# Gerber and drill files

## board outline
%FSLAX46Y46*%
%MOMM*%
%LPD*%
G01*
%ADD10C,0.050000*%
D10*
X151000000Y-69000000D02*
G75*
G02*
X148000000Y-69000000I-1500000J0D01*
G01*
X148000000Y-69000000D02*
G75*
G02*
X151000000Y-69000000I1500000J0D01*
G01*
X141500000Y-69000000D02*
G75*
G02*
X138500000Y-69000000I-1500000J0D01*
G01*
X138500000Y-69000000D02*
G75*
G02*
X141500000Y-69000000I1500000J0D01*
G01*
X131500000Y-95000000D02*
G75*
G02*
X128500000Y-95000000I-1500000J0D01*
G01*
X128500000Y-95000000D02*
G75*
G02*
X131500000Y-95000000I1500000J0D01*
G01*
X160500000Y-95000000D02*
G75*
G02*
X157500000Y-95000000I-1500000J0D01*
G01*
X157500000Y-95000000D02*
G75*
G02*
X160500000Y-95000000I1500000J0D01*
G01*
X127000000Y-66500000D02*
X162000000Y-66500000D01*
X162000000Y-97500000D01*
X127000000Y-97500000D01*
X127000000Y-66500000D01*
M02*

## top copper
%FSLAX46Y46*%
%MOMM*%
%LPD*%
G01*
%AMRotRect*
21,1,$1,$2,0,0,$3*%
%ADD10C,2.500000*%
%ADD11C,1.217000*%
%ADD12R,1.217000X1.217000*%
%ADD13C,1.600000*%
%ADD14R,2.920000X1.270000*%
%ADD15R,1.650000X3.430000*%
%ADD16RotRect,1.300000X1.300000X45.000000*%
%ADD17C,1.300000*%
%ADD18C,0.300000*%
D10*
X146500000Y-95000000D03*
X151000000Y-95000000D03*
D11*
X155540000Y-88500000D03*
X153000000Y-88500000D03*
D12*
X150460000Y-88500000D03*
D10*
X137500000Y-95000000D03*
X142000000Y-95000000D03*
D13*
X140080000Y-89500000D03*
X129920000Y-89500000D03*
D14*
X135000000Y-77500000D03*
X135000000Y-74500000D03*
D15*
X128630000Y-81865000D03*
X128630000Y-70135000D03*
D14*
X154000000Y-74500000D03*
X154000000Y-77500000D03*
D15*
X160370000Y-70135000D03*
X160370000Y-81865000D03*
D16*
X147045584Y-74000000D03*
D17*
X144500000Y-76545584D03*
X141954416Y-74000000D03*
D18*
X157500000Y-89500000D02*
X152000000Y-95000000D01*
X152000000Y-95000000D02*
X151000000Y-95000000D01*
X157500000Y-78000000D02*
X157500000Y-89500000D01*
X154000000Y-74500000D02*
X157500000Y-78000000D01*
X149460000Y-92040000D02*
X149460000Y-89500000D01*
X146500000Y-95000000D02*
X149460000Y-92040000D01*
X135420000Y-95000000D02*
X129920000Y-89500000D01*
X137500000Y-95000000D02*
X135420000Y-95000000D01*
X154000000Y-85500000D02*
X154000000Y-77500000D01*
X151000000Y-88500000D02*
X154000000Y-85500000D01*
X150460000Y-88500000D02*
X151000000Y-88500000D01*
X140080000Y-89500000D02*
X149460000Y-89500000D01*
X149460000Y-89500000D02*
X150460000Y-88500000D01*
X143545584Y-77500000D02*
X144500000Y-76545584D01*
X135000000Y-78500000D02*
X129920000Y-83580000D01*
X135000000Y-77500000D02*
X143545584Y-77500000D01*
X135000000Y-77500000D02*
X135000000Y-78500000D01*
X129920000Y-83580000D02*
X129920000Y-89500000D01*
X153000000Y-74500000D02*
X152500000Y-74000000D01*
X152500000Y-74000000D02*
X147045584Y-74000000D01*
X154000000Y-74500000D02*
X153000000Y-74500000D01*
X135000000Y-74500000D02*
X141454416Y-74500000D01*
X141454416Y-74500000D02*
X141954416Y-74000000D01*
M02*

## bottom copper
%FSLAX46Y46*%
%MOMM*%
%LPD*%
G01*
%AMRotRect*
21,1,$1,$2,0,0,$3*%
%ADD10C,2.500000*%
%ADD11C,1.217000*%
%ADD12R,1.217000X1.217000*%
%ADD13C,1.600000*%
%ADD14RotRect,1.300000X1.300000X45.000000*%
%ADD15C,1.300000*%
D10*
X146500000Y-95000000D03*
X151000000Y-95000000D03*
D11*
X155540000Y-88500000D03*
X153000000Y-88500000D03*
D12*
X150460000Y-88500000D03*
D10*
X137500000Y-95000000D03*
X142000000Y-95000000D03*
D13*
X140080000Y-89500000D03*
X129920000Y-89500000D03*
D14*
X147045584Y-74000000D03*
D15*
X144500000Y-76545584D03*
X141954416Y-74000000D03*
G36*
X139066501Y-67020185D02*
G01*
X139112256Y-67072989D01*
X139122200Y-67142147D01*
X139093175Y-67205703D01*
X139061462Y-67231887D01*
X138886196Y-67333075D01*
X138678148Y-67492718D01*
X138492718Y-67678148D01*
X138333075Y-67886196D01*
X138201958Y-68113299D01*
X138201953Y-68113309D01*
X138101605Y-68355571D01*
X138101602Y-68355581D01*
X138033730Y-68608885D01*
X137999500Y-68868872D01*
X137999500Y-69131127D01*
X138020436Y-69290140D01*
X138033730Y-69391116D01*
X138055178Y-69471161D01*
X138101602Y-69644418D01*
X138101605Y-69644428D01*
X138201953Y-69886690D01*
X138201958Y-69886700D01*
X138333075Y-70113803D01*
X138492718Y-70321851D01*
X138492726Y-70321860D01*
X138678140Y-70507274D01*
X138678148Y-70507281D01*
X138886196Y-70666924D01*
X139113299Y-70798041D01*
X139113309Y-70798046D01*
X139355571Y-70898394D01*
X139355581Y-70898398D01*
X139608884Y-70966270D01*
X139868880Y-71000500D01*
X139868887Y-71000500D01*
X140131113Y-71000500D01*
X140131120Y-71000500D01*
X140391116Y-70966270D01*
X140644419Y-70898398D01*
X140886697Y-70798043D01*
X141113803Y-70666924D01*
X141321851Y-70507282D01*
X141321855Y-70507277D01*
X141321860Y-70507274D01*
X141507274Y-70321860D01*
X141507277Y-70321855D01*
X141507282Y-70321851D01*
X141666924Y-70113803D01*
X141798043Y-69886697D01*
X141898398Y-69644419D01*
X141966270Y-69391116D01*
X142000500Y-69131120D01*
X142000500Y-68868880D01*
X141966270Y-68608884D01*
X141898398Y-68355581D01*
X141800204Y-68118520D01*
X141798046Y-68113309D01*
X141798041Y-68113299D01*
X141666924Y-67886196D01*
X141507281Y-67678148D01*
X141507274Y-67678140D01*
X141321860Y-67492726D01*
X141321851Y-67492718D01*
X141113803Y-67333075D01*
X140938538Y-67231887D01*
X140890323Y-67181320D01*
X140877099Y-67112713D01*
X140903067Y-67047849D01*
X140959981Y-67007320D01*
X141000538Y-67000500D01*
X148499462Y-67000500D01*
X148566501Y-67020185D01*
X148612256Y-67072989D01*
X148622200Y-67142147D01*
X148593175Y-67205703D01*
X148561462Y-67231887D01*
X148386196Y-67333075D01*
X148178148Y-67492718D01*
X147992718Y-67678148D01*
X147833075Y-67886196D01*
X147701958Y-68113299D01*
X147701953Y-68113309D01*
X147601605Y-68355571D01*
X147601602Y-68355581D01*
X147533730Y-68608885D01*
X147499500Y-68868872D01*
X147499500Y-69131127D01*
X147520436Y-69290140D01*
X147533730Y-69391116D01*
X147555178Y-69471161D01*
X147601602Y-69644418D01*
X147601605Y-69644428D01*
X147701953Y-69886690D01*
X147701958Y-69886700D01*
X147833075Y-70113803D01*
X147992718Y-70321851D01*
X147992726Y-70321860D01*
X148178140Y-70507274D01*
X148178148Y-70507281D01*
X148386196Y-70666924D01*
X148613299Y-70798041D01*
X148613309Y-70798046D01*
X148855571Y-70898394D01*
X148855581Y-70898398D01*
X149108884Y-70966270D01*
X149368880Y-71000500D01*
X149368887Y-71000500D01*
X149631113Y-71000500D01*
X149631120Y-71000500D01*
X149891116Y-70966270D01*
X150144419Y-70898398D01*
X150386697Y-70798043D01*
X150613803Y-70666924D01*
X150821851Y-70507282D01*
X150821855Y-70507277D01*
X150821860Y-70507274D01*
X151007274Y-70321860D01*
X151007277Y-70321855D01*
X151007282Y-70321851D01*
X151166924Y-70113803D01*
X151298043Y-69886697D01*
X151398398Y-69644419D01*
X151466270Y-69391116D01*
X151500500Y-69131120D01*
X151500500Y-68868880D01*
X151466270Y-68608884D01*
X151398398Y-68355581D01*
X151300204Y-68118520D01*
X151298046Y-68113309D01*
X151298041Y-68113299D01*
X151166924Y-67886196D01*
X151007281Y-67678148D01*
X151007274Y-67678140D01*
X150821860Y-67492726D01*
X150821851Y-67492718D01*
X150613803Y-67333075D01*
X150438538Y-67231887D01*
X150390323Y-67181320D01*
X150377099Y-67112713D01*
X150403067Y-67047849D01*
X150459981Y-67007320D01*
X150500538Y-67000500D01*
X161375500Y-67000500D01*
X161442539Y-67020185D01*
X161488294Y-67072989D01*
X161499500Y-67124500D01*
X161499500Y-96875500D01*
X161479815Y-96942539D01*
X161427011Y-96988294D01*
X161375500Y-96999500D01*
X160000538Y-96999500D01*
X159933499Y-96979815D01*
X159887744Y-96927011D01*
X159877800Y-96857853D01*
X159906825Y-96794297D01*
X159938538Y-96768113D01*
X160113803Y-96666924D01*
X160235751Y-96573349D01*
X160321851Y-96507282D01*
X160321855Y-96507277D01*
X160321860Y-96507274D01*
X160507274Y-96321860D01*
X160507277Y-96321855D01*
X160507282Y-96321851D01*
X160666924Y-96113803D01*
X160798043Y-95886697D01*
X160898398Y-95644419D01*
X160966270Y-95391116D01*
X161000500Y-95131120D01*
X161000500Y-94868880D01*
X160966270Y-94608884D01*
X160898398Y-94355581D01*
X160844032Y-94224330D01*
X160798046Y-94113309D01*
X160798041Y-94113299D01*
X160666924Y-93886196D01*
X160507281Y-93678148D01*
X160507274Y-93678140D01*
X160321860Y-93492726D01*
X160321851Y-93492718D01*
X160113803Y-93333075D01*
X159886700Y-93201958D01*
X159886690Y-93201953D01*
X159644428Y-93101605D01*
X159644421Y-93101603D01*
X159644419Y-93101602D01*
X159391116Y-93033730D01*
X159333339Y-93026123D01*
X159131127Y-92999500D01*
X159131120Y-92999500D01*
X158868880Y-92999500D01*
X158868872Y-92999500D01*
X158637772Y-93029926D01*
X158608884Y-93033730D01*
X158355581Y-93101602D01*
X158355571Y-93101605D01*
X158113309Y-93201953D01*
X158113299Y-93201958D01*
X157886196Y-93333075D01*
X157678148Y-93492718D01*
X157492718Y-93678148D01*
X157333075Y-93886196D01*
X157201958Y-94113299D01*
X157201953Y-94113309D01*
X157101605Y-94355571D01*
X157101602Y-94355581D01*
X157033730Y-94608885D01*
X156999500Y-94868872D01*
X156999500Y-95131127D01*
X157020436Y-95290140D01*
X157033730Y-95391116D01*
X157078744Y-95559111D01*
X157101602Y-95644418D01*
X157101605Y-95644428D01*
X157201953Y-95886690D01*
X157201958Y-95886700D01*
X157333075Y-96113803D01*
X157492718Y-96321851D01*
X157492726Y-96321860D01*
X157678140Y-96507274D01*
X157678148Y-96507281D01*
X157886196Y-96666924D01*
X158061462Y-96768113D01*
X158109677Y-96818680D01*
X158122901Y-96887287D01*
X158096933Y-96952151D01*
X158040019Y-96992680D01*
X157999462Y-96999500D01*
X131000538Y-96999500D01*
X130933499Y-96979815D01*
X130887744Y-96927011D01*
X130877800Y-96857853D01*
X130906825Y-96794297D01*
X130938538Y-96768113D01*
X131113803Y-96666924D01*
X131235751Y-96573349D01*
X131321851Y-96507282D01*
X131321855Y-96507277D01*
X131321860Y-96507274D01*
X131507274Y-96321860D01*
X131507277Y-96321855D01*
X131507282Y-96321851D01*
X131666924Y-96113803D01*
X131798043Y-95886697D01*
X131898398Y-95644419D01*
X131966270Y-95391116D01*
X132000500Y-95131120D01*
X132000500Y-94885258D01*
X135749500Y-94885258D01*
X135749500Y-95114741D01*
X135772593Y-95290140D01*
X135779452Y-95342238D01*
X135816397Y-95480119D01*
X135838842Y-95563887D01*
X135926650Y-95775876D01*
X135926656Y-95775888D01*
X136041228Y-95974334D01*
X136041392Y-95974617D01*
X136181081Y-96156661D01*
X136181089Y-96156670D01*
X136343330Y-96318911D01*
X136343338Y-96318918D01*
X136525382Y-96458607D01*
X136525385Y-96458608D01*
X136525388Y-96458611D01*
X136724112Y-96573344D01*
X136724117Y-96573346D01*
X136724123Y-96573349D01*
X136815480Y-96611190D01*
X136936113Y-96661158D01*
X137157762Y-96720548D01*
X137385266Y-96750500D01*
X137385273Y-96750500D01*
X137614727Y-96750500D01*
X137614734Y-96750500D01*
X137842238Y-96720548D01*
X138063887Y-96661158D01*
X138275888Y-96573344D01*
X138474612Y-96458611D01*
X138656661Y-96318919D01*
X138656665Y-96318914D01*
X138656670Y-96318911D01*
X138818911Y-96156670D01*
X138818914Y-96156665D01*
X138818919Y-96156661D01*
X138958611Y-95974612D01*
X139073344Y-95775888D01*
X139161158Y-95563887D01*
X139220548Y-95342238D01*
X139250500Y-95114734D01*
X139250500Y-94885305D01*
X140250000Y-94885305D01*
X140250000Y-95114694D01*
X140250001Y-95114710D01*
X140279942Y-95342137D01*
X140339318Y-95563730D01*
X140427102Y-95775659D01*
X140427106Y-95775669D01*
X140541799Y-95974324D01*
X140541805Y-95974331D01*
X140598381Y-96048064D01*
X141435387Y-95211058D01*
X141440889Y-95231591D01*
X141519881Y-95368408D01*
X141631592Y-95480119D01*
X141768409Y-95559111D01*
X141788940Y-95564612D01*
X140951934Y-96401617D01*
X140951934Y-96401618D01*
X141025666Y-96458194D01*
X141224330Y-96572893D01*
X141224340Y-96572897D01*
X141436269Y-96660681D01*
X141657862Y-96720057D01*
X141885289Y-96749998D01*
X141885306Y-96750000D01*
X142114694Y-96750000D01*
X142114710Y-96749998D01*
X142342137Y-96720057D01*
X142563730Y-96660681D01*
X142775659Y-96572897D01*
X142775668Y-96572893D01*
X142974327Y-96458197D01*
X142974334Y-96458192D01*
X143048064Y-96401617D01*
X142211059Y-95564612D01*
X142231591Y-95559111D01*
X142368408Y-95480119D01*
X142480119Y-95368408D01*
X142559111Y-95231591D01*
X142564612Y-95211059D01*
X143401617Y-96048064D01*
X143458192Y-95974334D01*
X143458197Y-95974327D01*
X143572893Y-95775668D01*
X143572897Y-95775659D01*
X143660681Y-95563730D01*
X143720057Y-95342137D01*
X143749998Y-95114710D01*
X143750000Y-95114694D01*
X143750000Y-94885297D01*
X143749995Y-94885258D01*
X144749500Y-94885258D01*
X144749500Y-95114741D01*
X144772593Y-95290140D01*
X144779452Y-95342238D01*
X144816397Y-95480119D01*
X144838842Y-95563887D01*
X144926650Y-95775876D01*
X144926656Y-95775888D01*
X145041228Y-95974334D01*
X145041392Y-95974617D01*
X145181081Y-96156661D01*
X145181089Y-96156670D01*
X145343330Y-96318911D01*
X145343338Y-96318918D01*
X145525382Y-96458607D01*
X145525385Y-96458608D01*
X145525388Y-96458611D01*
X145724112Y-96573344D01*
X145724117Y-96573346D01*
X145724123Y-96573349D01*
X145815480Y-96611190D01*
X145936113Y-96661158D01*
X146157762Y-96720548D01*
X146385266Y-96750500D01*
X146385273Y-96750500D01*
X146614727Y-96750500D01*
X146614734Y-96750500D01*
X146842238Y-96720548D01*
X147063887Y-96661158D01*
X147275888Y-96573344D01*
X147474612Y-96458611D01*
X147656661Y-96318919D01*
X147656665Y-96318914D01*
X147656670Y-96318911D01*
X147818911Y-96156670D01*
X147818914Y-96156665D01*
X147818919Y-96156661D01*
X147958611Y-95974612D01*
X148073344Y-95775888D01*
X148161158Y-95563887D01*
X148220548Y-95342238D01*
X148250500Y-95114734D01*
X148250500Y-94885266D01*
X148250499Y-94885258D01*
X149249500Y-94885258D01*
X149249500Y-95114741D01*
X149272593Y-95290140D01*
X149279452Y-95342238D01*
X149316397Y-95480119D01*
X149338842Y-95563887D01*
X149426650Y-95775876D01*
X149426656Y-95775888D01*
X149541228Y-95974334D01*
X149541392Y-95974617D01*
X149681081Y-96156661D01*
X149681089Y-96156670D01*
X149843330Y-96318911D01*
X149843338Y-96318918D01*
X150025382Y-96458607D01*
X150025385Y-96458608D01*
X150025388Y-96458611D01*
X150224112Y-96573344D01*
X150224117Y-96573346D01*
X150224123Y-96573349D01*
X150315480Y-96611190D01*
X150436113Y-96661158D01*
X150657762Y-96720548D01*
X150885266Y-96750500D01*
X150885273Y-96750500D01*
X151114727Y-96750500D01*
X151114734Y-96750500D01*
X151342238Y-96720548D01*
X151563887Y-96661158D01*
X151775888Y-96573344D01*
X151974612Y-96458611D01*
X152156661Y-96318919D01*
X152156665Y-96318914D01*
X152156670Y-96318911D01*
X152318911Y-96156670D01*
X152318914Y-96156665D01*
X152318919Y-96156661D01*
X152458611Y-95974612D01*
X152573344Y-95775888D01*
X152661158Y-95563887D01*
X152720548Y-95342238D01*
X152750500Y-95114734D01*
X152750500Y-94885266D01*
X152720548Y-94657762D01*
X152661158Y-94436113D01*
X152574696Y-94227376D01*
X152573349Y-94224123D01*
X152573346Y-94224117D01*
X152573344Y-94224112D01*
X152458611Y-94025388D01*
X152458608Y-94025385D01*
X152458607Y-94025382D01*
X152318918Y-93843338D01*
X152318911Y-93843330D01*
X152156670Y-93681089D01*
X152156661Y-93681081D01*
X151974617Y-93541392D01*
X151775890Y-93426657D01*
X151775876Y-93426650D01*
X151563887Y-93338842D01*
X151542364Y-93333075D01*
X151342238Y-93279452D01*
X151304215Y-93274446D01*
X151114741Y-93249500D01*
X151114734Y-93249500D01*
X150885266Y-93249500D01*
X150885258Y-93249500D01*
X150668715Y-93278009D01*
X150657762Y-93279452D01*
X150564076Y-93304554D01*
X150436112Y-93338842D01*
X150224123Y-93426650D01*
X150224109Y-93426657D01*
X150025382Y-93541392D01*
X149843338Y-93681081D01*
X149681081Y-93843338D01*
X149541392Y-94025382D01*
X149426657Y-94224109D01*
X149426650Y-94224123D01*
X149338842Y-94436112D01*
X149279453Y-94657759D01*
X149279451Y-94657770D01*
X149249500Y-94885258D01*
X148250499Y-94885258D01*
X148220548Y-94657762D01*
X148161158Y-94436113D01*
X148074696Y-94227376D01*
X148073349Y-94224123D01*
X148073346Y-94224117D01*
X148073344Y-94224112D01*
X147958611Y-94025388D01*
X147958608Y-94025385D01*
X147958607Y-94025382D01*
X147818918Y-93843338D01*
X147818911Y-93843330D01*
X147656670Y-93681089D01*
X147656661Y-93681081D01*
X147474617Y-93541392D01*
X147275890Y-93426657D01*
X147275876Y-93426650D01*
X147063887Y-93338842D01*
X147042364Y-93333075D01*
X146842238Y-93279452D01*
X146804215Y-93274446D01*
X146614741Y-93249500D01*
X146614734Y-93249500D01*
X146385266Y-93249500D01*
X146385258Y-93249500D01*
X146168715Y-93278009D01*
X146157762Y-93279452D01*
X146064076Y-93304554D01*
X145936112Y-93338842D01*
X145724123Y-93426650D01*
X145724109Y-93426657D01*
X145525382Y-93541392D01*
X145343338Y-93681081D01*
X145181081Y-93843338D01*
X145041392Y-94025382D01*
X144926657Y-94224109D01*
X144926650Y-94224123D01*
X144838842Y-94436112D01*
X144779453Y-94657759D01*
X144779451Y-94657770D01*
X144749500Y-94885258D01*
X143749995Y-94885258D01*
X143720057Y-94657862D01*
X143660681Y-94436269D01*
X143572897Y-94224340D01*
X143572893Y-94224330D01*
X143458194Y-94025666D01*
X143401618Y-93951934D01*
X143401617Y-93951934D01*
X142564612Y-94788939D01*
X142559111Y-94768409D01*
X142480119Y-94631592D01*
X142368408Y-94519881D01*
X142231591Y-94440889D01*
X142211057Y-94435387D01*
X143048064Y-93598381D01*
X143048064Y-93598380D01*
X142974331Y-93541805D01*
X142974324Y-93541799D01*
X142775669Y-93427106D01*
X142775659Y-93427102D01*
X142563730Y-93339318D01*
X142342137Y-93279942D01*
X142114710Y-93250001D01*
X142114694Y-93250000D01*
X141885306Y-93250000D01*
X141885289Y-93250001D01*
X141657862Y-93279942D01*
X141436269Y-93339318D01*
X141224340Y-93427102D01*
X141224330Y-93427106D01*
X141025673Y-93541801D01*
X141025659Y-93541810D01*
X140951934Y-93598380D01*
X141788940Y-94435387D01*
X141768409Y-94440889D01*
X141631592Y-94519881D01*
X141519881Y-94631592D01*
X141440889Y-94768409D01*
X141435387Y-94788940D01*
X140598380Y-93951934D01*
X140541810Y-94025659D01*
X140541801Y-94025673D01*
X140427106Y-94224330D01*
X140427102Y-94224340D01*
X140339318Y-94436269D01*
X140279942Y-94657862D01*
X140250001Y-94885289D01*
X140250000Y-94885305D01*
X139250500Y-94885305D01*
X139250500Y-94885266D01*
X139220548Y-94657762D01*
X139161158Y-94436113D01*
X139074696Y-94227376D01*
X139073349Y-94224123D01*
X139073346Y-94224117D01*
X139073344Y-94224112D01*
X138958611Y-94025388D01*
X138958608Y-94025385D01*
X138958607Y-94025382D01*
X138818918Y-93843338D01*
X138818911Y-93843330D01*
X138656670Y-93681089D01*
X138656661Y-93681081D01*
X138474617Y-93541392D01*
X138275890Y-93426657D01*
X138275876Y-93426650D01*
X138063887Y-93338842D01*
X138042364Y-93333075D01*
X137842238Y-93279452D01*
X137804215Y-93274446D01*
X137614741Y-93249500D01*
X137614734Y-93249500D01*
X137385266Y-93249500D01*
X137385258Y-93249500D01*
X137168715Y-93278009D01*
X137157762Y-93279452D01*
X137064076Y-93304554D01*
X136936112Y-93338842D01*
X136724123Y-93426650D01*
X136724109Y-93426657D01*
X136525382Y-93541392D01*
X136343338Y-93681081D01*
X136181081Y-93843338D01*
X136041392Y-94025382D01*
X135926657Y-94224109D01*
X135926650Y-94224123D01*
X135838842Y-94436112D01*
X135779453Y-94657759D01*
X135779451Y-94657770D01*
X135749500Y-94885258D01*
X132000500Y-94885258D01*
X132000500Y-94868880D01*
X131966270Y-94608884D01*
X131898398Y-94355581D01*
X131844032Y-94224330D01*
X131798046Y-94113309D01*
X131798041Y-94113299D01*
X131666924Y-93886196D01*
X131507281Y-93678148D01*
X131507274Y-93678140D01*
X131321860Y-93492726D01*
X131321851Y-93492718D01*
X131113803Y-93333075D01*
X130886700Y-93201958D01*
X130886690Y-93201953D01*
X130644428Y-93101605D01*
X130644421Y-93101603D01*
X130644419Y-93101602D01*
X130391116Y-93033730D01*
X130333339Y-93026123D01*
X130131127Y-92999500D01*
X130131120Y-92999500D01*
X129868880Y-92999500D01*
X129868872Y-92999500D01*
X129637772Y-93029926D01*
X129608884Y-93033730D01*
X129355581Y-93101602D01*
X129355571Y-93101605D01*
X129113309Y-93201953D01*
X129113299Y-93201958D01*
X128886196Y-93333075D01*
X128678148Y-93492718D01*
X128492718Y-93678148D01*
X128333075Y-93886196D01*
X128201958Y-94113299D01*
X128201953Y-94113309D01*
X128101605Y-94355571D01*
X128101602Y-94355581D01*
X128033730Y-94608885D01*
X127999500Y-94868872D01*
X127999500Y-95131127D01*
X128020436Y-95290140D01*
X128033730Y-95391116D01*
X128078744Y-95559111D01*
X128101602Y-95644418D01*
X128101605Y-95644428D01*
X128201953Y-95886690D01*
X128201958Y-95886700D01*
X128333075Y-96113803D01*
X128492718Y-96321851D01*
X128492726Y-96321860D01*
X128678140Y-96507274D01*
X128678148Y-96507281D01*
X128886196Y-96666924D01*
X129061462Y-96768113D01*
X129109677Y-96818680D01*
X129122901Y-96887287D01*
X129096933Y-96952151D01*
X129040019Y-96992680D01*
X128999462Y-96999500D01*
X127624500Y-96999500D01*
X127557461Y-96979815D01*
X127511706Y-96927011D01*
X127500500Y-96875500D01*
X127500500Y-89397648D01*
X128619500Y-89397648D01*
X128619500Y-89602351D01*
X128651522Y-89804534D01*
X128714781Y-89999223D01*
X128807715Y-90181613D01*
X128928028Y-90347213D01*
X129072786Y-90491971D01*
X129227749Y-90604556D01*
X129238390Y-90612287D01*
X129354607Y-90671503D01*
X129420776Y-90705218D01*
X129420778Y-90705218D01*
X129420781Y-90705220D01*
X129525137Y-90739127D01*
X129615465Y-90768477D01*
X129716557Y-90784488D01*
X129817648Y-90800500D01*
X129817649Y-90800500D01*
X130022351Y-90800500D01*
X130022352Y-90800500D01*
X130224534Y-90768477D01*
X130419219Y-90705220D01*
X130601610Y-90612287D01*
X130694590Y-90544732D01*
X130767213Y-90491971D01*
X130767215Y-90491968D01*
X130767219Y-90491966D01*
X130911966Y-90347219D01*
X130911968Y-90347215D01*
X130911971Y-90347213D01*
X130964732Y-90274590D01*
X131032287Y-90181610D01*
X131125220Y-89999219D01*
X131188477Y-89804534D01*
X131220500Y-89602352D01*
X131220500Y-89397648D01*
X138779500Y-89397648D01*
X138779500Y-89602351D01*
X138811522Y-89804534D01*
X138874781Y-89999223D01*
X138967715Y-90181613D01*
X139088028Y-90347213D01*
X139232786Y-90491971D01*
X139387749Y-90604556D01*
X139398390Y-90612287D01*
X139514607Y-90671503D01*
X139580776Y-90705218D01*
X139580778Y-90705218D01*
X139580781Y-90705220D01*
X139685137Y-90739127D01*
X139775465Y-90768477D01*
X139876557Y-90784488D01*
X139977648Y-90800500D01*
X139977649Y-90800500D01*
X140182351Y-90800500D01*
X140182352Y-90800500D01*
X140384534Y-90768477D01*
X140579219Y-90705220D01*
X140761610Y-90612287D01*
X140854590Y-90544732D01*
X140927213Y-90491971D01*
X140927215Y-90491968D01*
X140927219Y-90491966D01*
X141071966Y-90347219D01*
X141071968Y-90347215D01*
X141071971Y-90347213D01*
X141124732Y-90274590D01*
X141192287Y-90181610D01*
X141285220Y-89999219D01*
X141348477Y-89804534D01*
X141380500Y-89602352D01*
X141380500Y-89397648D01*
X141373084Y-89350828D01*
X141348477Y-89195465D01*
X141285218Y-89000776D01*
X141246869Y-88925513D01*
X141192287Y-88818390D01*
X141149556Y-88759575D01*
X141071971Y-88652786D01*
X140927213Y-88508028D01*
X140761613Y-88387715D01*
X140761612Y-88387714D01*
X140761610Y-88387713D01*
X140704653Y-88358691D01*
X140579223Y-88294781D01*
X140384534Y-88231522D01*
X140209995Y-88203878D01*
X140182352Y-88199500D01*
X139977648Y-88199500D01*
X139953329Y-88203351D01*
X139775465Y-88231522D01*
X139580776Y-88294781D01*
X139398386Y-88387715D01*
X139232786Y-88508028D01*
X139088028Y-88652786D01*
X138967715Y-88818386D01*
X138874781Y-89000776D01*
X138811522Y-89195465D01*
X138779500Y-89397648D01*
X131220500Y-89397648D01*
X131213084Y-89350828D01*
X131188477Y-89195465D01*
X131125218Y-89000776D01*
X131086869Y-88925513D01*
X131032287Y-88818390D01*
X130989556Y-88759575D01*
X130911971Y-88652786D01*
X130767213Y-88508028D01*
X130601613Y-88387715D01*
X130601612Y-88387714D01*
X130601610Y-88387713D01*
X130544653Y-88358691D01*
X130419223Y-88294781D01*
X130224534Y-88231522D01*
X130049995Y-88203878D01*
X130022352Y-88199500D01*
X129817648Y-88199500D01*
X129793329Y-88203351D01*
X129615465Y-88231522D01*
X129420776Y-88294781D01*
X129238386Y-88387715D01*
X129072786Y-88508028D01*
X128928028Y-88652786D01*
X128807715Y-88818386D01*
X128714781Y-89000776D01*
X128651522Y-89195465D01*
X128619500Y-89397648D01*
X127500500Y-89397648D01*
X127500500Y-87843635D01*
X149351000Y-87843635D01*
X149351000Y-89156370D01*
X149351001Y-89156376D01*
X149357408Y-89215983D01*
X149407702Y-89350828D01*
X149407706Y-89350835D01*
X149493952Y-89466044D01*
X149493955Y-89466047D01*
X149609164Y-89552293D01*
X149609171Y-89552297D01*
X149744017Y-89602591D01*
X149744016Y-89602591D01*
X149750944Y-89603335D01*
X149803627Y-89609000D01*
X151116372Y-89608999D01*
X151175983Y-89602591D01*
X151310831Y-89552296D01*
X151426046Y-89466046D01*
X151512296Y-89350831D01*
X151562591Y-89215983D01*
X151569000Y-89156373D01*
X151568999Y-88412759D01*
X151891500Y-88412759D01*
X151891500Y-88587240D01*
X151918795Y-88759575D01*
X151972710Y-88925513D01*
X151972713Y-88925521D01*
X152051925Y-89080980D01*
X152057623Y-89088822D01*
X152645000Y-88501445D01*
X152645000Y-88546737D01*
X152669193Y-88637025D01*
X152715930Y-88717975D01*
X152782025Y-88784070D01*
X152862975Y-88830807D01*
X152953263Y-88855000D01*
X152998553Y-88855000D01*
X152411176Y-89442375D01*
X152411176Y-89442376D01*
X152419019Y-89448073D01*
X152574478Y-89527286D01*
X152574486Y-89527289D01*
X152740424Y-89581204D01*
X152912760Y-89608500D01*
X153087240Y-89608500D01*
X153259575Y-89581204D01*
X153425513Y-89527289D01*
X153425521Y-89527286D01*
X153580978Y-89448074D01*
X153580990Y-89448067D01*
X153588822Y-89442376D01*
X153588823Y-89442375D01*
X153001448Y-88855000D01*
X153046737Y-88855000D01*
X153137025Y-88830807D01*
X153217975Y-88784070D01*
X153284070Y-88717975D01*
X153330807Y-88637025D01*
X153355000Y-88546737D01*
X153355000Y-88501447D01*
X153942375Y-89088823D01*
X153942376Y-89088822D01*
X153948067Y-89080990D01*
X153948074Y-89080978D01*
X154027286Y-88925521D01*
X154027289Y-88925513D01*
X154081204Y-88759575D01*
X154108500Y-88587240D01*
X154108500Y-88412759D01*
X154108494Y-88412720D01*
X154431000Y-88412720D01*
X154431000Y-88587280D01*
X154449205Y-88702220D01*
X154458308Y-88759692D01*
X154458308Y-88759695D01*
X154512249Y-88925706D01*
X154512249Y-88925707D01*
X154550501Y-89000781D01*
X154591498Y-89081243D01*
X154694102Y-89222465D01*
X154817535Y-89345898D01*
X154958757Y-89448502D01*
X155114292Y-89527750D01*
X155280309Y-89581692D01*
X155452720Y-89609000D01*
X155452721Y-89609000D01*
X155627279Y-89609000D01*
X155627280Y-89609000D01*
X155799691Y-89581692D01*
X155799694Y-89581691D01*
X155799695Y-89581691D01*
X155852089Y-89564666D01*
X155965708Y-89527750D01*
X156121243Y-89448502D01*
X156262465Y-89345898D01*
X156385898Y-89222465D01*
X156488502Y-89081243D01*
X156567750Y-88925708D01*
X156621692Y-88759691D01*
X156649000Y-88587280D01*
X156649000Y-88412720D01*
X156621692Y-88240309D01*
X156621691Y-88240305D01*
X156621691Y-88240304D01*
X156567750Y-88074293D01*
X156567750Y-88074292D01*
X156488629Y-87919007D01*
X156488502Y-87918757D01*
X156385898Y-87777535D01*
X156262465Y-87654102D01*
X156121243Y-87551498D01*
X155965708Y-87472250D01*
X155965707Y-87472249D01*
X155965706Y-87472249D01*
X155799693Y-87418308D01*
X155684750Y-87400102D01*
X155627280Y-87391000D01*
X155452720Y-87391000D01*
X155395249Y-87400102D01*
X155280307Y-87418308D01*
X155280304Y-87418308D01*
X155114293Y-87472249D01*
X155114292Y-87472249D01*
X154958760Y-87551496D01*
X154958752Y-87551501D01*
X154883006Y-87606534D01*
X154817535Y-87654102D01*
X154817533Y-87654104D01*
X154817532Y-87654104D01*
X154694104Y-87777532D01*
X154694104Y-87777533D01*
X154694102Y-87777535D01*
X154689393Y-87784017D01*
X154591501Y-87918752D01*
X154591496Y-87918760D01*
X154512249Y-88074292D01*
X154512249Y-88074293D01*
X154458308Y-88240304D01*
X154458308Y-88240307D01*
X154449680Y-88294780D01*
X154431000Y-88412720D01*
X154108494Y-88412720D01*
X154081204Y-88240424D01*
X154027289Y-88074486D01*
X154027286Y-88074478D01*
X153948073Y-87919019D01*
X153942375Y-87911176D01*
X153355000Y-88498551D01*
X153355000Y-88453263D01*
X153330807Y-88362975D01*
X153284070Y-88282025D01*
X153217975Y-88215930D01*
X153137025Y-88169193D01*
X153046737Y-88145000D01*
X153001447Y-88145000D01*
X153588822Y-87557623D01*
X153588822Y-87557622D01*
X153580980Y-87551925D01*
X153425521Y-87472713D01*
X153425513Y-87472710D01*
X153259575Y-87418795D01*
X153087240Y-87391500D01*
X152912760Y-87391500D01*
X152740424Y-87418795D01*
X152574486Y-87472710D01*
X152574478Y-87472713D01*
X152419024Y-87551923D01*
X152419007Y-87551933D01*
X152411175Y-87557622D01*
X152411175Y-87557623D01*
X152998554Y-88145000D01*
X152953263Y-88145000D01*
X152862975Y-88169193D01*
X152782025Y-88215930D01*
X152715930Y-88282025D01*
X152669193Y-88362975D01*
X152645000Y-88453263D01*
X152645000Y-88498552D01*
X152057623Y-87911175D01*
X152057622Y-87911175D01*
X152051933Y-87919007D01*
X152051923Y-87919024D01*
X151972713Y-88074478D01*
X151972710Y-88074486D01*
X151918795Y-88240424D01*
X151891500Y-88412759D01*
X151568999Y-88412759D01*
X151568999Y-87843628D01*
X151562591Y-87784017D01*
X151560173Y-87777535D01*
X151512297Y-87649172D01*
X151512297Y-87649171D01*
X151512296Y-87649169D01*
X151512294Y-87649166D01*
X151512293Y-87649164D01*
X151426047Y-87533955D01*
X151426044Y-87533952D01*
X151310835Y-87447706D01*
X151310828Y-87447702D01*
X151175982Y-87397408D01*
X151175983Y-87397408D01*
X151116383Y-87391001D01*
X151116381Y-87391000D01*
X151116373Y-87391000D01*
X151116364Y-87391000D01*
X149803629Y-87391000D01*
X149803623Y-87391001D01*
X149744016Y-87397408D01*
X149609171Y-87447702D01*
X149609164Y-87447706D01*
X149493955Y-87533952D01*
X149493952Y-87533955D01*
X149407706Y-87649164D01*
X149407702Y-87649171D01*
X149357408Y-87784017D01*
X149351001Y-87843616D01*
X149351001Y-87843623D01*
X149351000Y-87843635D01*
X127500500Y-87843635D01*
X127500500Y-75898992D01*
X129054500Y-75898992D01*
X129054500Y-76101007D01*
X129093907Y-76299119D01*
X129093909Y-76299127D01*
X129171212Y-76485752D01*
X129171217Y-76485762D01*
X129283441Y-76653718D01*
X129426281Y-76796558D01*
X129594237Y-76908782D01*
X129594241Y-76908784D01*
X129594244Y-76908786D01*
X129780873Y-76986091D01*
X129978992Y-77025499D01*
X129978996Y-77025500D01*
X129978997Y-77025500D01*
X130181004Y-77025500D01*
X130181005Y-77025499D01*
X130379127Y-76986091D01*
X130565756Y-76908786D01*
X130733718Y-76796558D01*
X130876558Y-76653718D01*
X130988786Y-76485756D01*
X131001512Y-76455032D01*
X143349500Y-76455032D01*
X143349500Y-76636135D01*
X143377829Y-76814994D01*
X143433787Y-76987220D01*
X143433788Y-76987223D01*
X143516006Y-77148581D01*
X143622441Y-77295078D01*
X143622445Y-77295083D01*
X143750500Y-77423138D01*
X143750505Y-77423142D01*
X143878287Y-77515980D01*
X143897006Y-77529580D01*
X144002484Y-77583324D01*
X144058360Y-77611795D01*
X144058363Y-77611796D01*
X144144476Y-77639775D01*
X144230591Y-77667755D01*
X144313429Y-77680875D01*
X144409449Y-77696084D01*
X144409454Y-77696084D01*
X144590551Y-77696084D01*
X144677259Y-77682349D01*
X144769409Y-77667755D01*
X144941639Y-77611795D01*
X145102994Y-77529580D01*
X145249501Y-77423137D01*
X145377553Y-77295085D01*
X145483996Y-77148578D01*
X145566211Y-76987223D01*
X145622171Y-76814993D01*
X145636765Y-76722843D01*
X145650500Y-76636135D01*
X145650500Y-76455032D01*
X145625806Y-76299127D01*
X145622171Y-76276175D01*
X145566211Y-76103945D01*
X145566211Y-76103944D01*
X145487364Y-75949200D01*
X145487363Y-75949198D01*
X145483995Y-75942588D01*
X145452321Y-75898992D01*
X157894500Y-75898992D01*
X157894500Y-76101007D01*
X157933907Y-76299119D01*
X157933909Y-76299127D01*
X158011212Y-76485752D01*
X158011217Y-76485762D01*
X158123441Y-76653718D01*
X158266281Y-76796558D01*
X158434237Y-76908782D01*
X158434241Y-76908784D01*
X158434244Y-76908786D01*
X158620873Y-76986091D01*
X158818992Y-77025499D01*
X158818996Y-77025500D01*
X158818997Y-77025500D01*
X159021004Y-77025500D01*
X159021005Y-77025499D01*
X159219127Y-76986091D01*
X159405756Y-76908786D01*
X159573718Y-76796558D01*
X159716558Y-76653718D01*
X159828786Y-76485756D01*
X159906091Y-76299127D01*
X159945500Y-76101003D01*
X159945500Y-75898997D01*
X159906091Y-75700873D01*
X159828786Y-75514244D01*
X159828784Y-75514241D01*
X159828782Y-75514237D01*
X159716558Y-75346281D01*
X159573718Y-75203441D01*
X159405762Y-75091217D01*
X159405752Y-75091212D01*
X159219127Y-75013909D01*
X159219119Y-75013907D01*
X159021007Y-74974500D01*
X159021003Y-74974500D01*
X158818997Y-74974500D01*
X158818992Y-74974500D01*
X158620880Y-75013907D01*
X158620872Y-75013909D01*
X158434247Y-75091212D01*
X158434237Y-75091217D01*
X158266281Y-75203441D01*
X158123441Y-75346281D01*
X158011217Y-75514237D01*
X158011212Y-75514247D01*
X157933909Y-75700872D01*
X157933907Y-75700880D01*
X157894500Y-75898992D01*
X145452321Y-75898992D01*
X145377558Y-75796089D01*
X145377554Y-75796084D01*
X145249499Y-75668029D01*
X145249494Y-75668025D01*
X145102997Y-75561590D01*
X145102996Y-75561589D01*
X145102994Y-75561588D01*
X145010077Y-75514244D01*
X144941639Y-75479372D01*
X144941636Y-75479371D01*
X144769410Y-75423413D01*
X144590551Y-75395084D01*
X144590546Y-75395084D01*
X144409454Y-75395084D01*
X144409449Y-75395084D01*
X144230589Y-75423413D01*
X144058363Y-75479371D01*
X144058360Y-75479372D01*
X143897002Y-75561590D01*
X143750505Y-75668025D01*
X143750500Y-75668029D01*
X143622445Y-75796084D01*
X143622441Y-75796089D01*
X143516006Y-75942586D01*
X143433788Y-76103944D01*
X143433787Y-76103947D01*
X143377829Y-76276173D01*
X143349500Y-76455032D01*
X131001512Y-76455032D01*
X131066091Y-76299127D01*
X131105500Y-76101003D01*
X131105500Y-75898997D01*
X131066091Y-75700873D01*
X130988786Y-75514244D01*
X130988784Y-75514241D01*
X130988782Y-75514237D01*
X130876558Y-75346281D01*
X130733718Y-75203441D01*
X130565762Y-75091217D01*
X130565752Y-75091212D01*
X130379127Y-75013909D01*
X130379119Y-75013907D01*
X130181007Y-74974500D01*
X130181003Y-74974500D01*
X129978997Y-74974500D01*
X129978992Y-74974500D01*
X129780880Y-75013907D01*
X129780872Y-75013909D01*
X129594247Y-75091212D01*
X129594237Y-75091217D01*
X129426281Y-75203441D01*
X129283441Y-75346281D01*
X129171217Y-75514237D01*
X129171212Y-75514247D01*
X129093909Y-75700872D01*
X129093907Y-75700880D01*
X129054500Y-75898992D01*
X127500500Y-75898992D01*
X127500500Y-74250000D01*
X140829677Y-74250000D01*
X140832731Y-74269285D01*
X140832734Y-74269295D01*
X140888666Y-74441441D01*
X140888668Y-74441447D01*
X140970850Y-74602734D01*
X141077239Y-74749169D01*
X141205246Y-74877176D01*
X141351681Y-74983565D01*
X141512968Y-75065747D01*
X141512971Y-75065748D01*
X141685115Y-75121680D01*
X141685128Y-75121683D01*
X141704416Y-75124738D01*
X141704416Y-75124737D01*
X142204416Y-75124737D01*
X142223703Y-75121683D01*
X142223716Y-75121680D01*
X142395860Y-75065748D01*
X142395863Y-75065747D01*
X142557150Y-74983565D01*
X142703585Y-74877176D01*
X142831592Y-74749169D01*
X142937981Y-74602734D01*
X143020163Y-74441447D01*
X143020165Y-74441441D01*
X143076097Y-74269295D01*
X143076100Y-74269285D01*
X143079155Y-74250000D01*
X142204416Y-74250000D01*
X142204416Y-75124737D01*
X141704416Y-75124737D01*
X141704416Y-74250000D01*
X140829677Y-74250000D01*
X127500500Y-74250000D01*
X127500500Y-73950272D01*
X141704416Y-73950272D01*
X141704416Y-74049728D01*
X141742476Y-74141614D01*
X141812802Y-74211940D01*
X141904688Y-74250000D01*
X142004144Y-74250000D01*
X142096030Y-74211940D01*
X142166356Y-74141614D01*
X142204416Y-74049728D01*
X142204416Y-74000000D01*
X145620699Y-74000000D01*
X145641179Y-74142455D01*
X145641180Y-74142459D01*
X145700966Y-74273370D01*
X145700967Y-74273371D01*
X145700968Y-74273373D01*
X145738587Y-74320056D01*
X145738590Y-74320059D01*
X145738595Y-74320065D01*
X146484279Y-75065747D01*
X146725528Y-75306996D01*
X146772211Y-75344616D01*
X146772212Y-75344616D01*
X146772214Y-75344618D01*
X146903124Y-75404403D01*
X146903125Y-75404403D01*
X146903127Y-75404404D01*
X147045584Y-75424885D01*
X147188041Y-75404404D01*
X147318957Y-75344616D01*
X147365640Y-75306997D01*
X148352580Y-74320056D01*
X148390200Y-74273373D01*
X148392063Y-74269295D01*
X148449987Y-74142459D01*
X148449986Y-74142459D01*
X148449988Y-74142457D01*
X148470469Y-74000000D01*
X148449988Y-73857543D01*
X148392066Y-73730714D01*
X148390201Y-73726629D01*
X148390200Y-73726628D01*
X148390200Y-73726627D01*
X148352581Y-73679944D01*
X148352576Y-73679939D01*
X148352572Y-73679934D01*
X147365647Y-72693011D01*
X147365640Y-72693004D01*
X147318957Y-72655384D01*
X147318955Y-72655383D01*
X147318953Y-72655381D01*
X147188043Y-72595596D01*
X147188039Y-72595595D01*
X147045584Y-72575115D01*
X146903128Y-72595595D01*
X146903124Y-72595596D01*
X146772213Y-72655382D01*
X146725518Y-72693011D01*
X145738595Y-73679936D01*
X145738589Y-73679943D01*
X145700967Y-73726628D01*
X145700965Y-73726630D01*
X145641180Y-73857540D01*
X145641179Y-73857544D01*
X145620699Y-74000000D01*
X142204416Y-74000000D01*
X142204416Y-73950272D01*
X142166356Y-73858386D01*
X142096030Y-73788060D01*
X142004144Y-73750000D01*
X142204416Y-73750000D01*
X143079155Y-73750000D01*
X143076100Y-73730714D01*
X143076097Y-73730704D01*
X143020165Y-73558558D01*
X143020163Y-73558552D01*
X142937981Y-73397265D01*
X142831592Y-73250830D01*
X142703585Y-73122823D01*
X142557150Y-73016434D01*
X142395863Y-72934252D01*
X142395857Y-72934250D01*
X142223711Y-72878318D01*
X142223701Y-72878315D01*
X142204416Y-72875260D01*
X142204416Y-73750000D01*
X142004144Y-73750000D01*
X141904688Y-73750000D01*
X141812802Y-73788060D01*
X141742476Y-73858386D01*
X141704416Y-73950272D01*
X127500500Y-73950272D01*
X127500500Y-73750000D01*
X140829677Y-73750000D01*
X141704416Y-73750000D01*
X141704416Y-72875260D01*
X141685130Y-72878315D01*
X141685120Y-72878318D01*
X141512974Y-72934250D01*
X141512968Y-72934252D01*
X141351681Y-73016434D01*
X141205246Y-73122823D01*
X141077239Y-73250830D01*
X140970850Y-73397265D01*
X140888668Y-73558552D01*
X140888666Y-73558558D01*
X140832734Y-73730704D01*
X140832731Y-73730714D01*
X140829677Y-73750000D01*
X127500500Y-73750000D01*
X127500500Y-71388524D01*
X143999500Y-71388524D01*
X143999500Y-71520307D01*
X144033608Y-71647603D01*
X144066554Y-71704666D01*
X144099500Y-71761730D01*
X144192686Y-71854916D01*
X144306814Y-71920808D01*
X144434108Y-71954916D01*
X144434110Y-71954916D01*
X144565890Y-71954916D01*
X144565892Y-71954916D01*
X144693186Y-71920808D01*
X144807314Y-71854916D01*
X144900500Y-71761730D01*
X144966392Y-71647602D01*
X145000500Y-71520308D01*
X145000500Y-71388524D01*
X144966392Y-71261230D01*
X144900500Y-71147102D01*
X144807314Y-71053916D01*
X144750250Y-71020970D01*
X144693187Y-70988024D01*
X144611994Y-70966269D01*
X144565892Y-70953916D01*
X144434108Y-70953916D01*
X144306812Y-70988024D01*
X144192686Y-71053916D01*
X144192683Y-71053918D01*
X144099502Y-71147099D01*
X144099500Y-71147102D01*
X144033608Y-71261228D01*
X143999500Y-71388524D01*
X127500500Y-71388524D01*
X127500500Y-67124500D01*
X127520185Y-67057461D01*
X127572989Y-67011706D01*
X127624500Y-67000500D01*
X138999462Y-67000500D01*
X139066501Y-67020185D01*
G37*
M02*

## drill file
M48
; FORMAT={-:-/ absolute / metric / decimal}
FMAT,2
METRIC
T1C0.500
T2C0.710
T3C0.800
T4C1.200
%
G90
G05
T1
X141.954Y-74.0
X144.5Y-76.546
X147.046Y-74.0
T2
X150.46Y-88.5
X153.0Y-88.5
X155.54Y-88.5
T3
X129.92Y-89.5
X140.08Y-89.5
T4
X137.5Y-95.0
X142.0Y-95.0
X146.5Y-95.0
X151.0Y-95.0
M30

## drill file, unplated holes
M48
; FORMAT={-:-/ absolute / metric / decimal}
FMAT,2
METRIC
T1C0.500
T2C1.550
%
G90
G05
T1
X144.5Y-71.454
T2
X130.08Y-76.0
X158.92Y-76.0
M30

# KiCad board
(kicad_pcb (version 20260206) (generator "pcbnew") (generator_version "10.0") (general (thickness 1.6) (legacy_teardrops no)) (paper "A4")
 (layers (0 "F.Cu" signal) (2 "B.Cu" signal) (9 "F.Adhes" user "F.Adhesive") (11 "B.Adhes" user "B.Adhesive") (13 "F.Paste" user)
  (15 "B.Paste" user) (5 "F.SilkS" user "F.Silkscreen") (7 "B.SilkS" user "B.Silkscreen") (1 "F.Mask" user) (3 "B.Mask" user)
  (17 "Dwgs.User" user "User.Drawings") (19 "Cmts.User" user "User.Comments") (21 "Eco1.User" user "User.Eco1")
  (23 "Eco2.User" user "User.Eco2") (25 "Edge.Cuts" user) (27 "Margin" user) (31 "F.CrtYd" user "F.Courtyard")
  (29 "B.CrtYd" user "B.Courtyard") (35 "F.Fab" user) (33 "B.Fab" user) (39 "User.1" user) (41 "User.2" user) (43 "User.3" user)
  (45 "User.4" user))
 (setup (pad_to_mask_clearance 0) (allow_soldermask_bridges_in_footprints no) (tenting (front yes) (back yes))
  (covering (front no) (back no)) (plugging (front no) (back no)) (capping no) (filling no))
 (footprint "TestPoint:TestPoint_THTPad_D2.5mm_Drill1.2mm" (layer "F.Cu") (at 137.5 95)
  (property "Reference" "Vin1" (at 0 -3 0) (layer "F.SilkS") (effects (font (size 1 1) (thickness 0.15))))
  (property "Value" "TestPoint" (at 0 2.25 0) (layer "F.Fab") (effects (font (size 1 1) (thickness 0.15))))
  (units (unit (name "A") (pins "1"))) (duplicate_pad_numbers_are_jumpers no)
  (pad "1" thru_hole circle (at 0 0) (size 2.5 2.5) (drill 1.2) (layers "*.Cu" "*.Mask") (remove_unused_layers no) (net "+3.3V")))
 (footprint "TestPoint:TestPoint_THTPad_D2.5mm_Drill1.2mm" (layer "F.Cu") (at 142 95)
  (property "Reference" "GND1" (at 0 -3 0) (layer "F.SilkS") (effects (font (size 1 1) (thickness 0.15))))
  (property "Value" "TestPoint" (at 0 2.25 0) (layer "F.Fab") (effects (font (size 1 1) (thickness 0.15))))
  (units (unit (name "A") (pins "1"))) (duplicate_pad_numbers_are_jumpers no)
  (pad "1" thru_hole circle (at 0 0) (size 2.5 2.5) (drill 1.2) (layers "*.Cu" "*.Mask") (remove_unused_layers no) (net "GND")))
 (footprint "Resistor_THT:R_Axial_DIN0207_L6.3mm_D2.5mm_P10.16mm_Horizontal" (layer "F.Cu") (at 140.08 89.5 180)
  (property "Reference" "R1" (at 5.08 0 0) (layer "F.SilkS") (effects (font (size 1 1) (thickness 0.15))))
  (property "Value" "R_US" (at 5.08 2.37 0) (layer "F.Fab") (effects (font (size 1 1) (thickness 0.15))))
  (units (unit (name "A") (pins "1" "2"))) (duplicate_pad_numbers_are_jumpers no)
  (pad "1" thru_hole circle (at 0 0 180) (size 1.6 1.6) (drill 0.8) (layers "*.Cu" "*.Mask") (remove_unused_layers no) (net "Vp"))
  (pad "2" thru_hole circle (at 10.16 0 180) (size 1.6 1.6) (drill 0.8) (layers "*.Cu" "*.Mask") (remove_unused_layers no) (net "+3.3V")))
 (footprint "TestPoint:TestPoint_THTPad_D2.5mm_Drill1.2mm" (layer "F.Cu") (at 151 95)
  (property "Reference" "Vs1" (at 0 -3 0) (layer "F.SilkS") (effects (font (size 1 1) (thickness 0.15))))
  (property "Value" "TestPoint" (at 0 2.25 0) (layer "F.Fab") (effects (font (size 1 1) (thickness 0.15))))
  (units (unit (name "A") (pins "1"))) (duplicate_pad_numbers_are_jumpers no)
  (pad "1" thru_hole circle (at 0 0) (size 2.5 2.5) (drill 1.2) (layers "*.Cu" "*.Mask") (remove_unused_layers no) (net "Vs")))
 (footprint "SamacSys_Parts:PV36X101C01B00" (layer "F.Cu") (at 150.46 88.5 -90)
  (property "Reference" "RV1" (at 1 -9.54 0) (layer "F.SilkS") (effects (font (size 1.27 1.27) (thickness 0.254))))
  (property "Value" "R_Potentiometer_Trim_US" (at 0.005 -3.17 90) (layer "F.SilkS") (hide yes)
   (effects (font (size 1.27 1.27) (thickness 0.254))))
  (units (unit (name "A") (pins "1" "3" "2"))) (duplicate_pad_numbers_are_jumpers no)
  (pad "1" thru_hole rect (at 0 0 270) (size 1.217 1.217) (drill 0.71) (layers "*.Cu" "*.Mask") (remove_unused_layers no) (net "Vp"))
  (pad "2" thru_hole circle (at 0 -2.54 270) (size 1.217 1.217) (drill 0.71) (layers "*.Cu" "*.Mask") (remove_unused_layers no) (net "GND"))
  (pad "3" thru_hole circle (at 0 -5.08 270) (size 1.217 1.217) (drill 0.71) (layers "*.Cu" "*.Mask") (remove_unused_layers no)
   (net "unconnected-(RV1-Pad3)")))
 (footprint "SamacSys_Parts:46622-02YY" (layer "F.Cu") (at 135 76 -90)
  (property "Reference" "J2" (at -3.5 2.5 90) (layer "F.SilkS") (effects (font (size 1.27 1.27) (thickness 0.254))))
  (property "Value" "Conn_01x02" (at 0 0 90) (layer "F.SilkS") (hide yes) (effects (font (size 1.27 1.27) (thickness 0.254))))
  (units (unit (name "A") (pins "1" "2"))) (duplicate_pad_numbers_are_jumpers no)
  (pad "" np_thru_hole circle (at 0 4.92 270) (size 1.55 1.55) (drill 1.55) (layers "*.Cu" "*.Mask"))
  (pad "1" smd rect (at 1.5 0 270) (size 1.27 2.92) (layers "F.Cu" "F.Mask" "F.Paste") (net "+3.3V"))
  (pad "2" smd rect (at -1.5 0 270) (size 1.27 2.92) (layers "F.Cu" "F.Mask" "F.Paste") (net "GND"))
  (pad "3" smd rect (at 5.865 6.37) (size 1.65 3.43) (layers "F.Cu" "F.Mask" "F.Paste"))
  (pad "4" smd rect (at -5.865 6.37) (size 1.65 3.43) (layers "F.Cu" "F.Mask" "F.Paste")))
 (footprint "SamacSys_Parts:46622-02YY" (layer "F.Cu") (at 154 76 90)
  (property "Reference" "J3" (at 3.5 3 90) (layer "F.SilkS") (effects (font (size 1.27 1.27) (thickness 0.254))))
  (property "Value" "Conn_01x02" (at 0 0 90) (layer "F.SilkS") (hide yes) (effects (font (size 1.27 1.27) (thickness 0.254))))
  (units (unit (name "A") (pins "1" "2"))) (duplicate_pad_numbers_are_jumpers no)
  (pad "" np_thru_hole circle (at 0 4.92 90) (size 1.55 1.55) (drill 1.55) (layers "*.Cu" "*.Mask"))
  (pad "1" smd rect (at 1.5 0 90) (size 1.27 2.92) (layers "F.Cu" "F.Mask" "F.Paste") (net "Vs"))
  (pad "2" smd rect (at -1.5 0 90) (size 1.27 2.92) (layers "F.Cu" "F.Mask" "F.Paste") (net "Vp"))
  (pad "3" smd rect (at 5.865 6.37 180) (size 1.65 3.43) (layers "F.Cu" "F.Mask" "F.Paste"))
  (pad "4" smd rect (at -5.865 6.37 180) (size 1.65 3.43) (layers "F.Cu" "F.Mask" "F.Paste")))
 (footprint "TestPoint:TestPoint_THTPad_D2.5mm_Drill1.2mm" (layer "F.Cu") (at 146.5 95)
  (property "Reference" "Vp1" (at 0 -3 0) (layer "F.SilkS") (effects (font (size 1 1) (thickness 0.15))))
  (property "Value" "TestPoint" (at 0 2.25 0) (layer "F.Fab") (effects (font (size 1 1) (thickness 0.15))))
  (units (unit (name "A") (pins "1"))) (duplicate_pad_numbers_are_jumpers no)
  (pad "1" thru_hole circle (at 0 0) (size 2.5 2.5) (drill 1.2) (layers "*.Cu" "*.Mask") (remove_unused_layers no) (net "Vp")))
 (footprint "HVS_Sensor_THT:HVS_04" (layer "B.Cu") (at 144.5 74)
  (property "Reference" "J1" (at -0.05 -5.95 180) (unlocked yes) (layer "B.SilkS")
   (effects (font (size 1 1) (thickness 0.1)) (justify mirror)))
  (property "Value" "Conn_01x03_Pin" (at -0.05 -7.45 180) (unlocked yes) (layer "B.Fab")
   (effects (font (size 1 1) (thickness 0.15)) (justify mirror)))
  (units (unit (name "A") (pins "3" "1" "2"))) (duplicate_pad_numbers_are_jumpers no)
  (pad "" np_thru_hole circle (at 0 -2.545584 45) (size 0.5 0.5) (drill 0.5) (layers "*.Cu" "*.Mask"))
  (pad "1" thru_hole rect (at 2.545584 0 45) (size 1.3 1.3) (drill 0.5) (layers "*.Cu" "*.Mask") (remove_unused_layers no) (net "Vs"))
  (pad "2" thru_hole circle (at 0 2.545584 45) (size 1.3 1.3) (drill 0.5) (layers "*.Cu" "*.Mask") (remove_unused_layers no) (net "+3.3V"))
  (pad "3" thru_hole circle (at -2.545584 0 45) (size 1.3 1.3) (drill 0.5) (layers "*.Cu" "*.Mask") (remove_unused_layers no) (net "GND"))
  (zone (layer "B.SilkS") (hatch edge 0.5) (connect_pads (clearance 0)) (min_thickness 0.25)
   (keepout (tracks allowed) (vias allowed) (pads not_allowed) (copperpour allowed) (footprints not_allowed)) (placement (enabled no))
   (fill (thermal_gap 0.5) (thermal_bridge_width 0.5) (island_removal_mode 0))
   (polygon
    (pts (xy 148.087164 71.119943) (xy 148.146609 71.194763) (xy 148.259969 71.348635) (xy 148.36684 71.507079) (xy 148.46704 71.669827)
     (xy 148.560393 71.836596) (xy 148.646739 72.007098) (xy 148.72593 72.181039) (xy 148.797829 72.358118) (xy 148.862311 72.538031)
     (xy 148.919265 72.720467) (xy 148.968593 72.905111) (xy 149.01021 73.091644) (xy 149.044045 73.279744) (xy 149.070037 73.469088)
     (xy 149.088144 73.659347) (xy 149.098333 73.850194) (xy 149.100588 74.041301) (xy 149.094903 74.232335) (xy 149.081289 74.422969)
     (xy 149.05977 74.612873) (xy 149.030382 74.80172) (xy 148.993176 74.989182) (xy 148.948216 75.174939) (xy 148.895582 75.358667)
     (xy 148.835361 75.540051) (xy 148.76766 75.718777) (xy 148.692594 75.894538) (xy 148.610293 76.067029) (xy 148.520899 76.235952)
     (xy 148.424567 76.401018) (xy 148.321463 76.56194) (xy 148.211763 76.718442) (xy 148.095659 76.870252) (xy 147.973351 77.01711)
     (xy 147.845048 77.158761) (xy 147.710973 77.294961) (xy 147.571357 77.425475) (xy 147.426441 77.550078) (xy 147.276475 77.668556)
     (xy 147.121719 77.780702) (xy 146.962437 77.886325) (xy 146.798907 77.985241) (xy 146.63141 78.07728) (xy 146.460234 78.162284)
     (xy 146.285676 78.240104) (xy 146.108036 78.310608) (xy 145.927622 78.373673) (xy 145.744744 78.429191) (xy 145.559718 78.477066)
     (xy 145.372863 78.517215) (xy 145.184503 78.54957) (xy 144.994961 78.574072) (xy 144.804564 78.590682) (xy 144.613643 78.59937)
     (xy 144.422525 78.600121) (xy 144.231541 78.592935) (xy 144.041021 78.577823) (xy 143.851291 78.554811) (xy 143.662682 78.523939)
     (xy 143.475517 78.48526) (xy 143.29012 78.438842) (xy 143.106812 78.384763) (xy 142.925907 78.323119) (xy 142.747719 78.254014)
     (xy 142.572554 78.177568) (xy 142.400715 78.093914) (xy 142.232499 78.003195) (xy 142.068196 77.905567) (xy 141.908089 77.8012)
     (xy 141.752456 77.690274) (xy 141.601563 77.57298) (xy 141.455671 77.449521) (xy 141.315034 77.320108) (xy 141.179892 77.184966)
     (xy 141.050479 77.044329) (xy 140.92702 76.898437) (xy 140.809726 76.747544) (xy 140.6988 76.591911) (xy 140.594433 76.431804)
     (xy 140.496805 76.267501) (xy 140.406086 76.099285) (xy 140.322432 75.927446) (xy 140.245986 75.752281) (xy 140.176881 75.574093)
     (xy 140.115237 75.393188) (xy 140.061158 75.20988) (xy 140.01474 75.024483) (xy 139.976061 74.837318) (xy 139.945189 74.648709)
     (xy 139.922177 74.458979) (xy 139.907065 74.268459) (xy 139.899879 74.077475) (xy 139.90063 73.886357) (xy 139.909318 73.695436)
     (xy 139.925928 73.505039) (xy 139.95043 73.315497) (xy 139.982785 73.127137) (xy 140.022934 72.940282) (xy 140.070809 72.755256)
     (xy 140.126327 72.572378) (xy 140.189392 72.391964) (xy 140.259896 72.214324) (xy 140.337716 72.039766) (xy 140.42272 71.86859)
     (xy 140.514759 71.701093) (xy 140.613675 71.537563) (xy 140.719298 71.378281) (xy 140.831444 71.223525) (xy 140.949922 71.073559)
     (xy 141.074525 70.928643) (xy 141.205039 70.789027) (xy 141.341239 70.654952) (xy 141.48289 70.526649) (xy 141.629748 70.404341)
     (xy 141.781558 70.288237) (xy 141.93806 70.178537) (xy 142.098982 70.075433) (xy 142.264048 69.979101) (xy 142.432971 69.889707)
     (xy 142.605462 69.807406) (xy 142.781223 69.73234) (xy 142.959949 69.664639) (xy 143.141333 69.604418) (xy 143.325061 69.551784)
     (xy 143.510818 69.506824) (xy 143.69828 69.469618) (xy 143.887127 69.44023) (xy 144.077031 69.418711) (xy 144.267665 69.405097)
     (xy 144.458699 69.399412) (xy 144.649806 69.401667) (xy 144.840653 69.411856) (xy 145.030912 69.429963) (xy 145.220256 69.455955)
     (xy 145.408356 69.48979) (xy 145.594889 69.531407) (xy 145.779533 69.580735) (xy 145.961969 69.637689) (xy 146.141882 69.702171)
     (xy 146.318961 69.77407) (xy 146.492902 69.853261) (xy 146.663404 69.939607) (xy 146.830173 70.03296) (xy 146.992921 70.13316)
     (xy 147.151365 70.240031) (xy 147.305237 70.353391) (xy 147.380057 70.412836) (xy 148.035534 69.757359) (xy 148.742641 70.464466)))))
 (gr_rect (start 127 66.5) (end 162 97.5) (stroke (width 0.05) (type default)) (fill no) (layer "Edge.Cuts"))
 (gr_circle (center 130 95) (end 131.5 95) (stroke (width 0.05) (type default)) (fill no) (layer "Edge.Cuts"))
 (gr_circle (center 140 69) (end 141.5 69) (stroke (width 0.05) (type default)) (fill no) (layer "Edge.Cuts"))
 (gr_circle (center 149.5 69) (end 151 69) (stroke (width 0.05) (type default)) (fill no) (layer "Edge.Cuts"))
 (gr_circle (center 159 95) (end 160.5 95) (stroke (width 0.05) (type default)) (fill no) (layer "Edge.Cuts"))
 (segment (start 143.545584 77.5) (end 144.5 76.545584) (width 0.3) (layer "F.Cu") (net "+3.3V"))
 (segment (start 135 78.5) (end 129.92 83.58) (width 0.3) (layer "F.Cu") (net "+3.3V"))
 (segment (start 135 77.5) (end 143.545584 77.5) (width 0.3) (layer "F.Cu") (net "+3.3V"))
 (segment (start 137.5 95) (end 135.42 95) (width 0.3) (layer "F.Cu") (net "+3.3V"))
 (segment (start 135 77.5) (end 135 78.5) (width 0.3) (layer "F.Cu") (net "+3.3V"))
 (segment (start 129.92 83.58) (end 129.92 89.5) (width 0.3) (layer "F.Cu") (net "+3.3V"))
 (segment (start 135.42 95) (end 129.92 89.5) (width 0.3) (layer "F.Cu") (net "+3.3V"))
 (segment (start 135 74.5) (end 141.454416 74.5) (width 0.3) (layer "F.Cu") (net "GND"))
 (segment (start 141.454416 74.5) (end 141.954416 74) (width 0.3) (layer "F.Cu") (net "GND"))
 (segment (start 149.46 89.5) (end 150.46 88.5) (width 0.3) (layer "F.Cu") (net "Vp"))
 (segment (start 150.46 88.5) (end 151 88.5) (width 0.3) (layer "F.Cu") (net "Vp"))
 (segment (start 149.46 92.04) (end 149.46 89.5) (width 0.3) (layer "F.Cu") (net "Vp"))
 (segment (start 151 88.5) (end 154 85.5) (width 0.3) (layer "F.Cu") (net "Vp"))
 (segment (start 154 85.5) (end 154 77.5) (width 0.3) (layer "F.Cu") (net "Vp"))
 (segment (start 140.08 89.5) (end 149.46 89.5) (width 0.3) (layer "F.Cu") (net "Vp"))
 (segment (start 146.5 95) (end 149.46 92.04) (width 0.3) (layer "F.Cu") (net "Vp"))
 (segment (start 153 74.5) (end 152.5 74) (width 0.3) (layer "F.Cu") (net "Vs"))
 (segment (start 154 74.5) (end 157.5 78) (width 0.3) (layer "F.Cu") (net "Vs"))
 (segment (start 152.5 74) (end 147.045584 74) (width 0.3) (layer "F.Cu") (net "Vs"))
 (segment (start 154 74.5) (end 153 74.5) (width 0.3) (layer "F.Cu") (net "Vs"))
 (segment (start 157.5 78) (end 157.5 89.5) (width 0.3) (layer "F.Cu") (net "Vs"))
 (segment (start 157.5 89.5) (end 152 95) (width 0.3) (layer "F.Cu") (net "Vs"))
 (segment (start 152 95) (end 151 95) (width 0.3) (layer "F.Cu") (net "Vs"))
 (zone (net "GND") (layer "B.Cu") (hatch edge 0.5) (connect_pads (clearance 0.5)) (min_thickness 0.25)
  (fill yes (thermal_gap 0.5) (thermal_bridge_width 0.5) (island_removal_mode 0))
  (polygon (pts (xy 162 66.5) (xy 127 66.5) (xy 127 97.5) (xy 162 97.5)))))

